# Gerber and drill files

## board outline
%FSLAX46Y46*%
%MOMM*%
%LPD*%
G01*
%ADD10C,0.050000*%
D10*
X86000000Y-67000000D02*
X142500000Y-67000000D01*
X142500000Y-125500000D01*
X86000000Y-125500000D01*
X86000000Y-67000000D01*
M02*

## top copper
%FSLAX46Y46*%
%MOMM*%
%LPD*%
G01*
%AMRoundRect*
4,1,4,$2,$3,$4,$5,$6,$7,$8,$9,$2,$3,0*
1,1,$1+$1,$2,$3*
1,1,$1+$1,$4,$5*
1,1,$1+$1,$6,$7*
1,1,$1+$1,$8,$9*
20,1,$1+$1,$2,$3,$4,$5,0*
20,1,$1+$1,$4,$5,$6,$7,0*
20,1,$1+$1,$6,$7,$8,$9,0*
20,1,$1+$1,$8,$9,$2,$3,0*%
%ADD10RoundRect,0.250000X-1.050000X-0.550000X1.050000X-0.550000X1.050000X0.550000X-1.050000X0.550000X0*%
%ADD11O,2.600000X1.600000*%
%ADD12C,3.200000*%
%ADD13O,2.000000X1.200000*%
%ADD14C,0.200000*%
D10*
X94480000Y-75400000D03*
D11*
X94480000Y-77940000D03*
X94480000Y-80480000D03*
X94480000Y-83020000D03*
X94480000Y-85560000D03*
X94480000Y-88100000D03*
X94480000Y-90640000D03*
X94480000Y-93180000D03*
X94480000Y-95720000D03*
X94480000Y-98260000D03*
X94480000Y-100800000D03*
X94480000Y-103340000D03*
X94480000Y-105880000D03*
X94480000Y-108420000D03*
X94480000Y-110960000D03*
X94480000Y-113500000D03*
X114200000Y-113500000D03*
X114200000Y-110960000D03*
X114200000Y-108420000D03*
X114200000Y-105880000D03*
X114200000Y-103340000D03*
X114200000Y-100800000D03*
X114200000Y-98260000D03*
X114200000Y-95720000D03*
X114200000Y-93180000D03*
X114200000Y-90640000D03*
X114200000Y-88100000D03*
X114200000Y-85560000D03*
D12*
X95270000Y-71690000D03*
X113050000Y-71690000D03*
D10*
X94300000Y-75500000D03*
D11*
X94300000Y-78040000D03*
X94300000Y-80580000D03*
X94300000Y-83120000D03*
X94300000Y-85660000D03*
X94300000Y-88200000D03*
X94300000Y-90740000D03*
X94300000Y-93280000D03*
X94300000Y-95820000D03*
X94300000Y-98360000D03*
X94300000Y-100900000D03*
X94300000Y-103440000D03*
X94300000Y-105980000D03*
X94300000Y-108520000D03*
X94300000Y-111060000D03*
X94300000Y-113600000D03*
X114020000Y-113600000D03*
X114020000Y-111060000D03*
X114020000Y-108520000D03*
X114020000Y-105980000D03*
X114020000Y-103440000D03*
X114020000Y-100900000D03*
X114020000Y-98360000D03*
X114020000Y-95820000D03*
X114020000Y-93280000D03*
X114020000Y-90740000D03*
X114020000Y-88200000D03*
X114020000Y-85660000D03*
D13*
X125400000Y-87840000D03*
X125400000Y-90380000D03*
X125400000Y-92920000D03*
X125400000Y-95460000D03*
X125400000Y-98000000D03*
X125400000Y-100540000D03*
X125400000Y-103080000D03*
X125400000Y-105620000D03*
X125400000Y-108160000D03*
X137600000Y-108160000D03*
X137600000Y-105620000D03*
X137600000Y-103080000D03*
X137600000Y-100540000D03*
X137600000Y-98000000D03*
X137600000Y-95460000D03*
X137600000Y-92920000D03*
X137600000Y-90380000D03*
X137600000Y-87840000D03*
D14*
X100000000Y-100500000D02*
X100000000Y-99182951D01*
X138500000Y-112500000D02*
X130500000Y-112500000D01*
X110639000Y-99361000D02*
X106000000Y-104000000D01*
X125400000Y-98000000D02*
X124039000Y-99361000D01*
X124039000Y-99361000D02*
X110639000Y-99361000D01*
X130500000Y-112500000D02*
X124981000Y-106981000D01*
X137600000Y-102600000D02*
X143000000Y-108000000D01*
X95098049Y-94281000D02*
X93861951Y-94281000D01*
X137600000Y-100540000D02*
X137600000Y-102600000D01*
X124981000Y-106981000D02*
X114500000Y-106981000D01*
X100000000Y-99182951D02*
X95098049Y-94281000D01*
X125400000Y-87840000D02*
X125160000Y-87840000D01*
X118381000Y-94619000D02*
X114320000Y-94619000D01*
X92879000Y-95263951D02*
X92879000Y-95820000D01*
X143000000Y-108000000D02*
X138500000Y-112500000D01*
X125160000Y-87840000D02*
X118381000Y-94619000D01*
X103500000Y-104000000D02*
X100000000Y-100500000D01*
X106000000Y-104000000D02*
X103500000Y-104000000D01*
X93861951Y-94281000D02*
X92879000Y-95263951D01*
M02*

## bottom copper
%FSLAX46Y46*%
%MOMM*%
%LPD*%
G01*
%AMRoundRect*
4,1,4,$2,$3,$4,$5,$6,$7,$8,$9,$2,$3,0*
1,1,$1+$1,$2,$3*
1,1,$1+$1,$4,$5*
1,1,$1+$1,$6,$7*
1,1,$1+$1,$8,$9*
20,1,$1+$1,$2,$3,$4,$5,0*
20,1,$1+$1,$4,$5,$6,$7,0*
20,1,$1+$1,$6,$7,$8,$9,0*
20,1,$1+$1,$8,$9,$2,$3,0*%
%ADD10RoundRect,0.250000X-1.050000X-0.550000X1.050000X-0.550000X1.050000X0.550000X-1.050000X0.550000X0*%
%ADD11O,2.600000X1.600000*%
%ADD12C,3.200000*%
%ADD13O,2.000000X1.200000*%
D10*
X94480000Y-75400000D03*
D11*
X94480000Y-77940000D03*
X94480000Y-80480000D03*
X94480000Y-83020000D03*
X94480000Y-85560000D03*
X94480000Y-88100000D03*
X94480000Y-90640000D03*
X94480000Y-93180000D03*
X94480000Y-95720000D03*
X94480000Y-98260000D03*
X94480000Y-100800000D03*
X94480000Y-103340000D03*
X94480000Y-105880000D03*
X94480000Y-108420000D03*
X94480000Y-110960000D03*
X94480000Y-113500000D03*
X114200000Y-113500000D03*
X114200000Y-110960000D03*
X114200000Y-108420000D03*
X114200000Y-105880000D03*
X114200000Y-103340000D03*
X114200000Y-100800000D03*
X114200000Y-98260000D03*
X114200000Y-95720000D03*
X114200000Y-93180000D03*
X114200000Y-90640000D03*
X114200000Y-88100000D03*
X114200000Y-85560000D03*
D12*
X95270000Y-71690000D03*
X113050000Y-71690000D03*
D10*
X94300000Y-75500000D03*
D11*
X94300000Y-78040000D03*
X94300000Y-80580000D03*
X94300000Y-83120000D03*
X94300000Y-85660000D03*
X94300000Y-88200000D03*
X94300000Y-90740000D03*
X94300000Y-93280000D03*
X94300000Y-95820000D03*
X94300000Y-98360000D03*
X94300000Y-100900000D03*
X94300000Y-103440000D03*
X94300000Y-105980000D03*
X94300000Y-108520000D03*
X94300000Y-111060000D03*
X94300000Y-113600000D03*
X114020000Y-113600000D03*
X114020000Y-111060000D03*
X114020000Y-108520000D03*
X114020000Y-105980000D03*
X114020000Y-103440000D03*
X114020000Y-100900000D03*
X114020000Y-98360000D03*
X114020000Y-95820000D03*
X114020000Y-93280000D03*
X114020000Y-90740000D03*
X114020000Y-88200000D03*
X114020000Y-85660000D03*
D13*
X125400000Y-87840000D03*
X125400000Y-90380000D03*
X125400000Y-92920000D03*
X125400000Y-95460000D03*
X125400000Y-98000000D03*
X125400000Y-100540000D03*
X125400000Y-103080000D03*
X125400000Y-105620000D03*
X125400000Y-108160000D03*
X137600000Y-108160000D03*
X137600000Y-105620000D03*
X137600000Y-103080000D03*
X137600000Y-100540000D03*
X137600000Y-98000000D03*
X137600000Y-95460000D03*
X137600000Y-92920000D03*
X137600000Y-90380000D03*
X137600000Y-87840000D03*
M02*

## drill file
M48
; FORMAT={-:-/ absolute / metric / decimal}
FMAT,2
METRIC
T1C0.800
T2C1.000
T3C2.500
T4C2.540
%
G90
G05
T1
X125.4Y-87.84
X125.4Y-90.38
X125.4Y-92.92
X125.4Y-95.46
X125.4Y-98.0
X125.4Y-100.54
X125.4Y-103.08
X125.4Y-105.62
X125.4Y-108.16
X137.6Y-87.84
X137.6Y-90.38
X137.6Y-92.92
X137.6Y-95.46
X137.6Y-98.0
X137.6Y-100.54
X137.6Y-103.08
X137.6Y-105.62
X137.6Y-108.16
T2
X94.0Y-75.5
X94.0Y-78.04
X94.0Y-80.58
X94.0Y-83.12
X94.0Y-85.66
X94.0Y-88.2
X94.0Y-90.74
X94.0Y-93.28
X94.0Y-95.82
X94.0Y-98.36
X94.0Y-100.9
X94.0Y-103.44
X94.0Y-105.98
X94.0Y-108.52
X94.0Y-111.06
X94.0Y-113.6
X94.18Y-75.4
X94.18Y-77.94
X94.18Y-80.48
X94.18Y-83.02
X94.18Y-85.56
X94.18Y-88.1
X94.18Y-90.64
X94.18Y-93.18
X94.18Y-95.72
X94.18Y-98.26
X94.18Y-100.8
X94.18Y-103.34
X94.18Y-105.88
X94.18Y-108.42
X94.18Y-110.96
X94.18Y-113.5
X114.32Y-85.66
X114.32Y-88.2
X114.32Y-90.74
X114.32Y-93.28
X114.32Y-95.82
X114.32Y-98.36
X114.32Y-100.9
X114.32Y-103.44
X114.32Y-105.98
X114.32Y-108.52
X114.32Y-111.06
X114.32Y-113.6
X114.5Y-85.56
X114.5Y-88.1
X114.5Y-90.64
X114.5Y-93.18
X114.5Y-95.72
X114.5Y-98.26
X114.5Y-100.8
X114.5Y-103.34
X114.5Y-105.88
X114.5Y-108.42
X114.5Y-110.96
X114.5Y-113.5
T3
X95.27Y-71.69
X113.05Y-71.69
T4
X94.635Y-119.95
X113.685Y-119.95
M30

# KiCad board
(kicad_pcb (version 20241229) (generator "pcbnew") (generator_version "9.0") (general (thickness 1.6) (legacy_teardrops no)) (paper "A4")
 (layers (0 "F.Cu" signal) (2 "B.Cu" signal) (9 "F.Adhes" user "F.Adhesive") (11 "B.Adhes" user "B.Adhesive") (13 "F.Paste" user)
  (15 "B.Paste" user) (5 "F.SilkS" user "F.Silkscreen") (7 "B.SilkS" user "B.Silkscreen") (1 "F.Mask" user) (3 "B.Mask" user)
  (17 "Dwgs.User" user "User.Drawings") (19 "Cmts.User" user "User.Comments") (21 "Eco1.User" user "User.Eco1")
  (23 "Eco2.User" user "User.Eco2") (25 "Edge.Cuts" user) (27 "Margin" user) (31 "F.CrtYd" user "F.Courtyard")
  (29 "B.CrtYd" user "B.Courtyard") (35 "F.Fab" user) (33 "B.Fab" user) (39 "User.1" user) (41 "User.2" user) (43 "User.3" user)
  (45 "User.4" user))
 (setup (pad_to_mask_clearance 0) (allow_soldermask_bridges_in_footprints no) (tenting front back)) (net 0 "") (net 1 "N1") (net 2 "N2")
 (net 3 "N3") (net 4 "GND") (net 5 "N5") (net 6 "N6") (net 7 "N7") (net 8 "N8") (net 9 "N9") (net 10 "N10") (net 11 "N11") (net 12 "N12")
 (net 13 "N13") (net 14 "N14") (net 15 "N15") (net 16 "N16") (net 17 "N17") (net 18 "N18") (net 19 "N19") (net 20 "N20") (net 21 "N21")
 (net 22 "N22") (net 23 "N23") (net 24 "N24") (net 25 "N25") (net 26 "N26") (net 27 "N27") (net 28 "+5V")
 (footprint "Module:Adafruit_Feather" (layer "F.Cu") (at 94.18 75.4)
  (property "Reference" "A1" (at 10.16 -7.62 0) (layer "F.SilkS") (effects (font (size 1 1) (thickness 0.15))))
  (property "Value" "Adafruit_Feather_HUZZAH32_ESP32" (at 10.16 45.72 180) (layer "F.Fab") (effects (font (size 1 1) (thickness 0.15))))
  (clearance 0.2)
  (pad "1" thru_hole roundrect (at 0 0) (size 2.6 1.6) (drill 1 (offset 0.3 0)) (layers "*.Cu" "*.Mask") (remove_unused_layers no)
   (roundrect_rratio 0.15625) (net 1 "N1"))
  (pad "2" thru_hole oval (at 0 2.54) (size 2.6 1.6) (drill 1 (offset 0.3 0)) (layers "*.Cu" "*.Mask") (remove_unused_layers no)
   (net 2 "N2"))
  (pad "3" thru_hole oval (at 0 5.08) (size 2.6 1.6) (drill 1 (offset 0.3 0)) (layers "*.Cu" "*.Mask") (remove_unused_layers no)
   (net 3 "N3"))
  (pad "4" thru_hole oval (at 0 7.62) (size 2.6 1.6) (drill 1 (offset 0.3 0)) (layers "*.Cu" "*.Mask") (remove_unused_layers no)
   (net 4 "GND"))
  (pad "5" thru_hole oval (at 0 10.16) (size 2.6 1.6) (drill 1 (offset 0.3 0)) (layers "*.Cu" "*.Mask") (remove_unused_layers no)
   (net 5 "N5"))
  (pad "6" thru_hole oval (at 0 12.7) (size 2.6 1.6) (drill 1 (offset 0.3 0)) (layers "*.Cu" "*.Mask") (remove_unused_layers no)
   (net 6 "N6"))
  (pad "7" thru_hole oval (at 0 15.24) (size 2.6 1.6) (drill 1 (offset 0.3 0)) (layers "*.Cu" "*.Mask") (remove_unused_layers no)
   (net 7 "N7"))
  (pad "8" thru_hole oval (at 0 17.78) (size 2.6 1.6) (drill 1 (offset 0.3 0)) (layers "*.Cu" "*.Mask") (remove_unused_layers no)
   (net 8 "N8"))
  (pad "9" thru_hole oval (at 0 20.32) (size 2.6 1.6) (drill 1 (offset 0.3 0)) (layers "*.Cu" "*.Mask") (remove_unused_layers no)
   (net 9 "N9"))
  (pad "10" thru_hole oval (at 0 22.86) (size 2.6 1.6) (drill 1 (offset 0.3 0)) (layers "*.Cu" "*.Mask") (remove_unused_layers no)
   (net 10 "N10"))
  (pad "11" thru_hole oval (at 0 25.4) (size 2.6 1.6) (drill 1 (offset 0.3 0)) (layers "*.Cu" "*.Mask") (remove_unused_layers no)
   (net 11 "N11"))
  (pad "12" thru_hole oval (at 0 27.94) (size 2.6 1.6) (drill 1 (offset 0.3 0)) (layers "*.Cu" "*.Mask") (remove_unused_layers no)
   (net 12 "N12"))
  (pad "13" thru_hole oval (at 0 30.48) (size 2.6 1.6) (drill 1 (offset 0.3 0)) (layers "*.Cu" "*.Mask") (remove_unused_layers no)
   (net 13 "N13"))
  (pad "14" thru_hole oval (at 0 33.02) (size 2.6 1.6) (drill 1 (offset 0.3 0)) (layers "*.Cu" "*.Mask") (remove_unused_layers no)
   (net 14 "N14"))
  (pad "15" thru_hole oval (at 0 35.56) (size 2.6 1.6) (drill 1 (offset 0.3 0)) (layers "*.Cu" "*.Mask") (remove_unused_layers no)
   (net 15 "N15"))
  (pad "16" thru_hole oval (at 0 38.1) (size 2.6 1.6) (drill 1 (offset 0.3 0)) (layers "*.Cu" "*.Mask") (remove_unused_layers no)
   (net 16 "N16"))
  (pad "17" thru_hole oval (at 20.32 38.1 180) (size 2.6 1.6) (drill 1 (offset 0.3 0)) (layers "*.Cu" "*.Mask") (remove_unused_layers no)
   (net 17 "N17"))
  (pad "18" thru_hole oval (at 20.32 35.56 180) (size 2.6 1.6) (drill 1 (offset 0.3 0)) (layers "*.Cu" "*.Mask") (remove_unused_layers no)
   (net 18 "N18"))
  (pad "19" thru_hole oval (at 20.32 33.02 180) (size 2.6 1.6) (drill 1 (offset 0.3 0)) (layers "*.Cu" "*.Mask") (remove_unused_layers no)
   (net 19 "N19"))
  (pad "20" thru_hole oval (at 20.32 30.48 180) (size 2.6 1.6) (drill 1 (offset 0.3 0)) (layers "*.Cu" "*.Mask") (remove_unused_layers no)
   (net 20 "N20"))
  (pad "21" thru_hole oval (at 20.32 27.94 180) (size 2.6 1.6) (drill 1 (offset 0.3 0)) (layers "*.Cu" "*.Mask") (remove_unused_layers no)
   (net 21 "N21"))
  (pad "22" thru_hole oval (at 20.32 25.4 180) (size 2.6 1.6) (drill 1 (offset 0.3 0)) (layers "*.Cu" "*.Mask") (remove_unused_layers no)
   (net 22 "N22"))
  (pad "23" thru_hole oval (at 20.32 22.86 180) (size 2.6 1.6) (drill 1 (offset 0.3 0)) (layers "*.Cu" "*.Mask") (remove_unused_layers no)
   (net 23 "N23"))
  (pad "24" thru_hole oval (at 20.32 20.32 180) (size 2.6 1.6) (drill 1 (offset 0.3 0)) (layers "*.Cu" "*.Mask") (remove_unused_layers no)
   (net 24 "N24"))
  (pad "25" thru_hole oval (at 20.32 17.78 180) (size 2.6 1.6) (drill 1 (offset 0.3 0)) (layers "*.Cu" "*.Mask") (remove_unused_layers no)
   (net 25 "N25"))
  (pad "26" thru_hole oval (at 20.32 15.24 180) (size 2.6 1.6) (drill 1 (offset 0.3 0)) (layers "*.Cu" "*.Mask") (remove_unused_layers no)
   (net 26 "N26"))
  (pad "27" thru_hole oval (at 20.32 12.7 180) (size 2.6 1.6) (drill 1 (offset 0.3 0)) (layers "*.Cu" "*.Mask") (remove_unused_layers no)
   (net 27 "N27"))
  (pad "28" thru_hole oval (at 20.32 10.16 180) (size 2.6 1.6) (drill 1 (offset 0.3 0)) (layers "*.Cu" "*.Mask") (remove_unused_layers no)
   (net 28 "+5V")))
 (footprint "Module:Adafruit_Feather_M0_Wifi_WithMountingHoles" (layer "F.Cu") (at 94 75.5)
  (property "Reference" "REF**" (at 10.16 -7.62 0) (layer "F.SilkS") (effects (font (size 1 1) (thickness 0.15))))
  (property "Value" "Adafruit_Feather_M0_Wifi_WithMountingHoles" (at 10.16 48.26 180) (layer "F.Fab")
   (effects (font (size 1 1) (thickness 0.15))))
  (pad "" np_thru_hole circle (at 0.635 44.45 270) (size 2.54 2.54) (drill 2.54) (layers "*.Cu" "*.Mask"))
  (pad "" np_thru_hole circle (at 1.27 -3.81 270) (size 3.2 3.2) (drill 2.5) (layers "*.Cu" "*.Mask"))
  (pad "" np_thru_hole circle (at 19.05 -3.81 270) (size 3.2 3.2) (drill 2.5) (layers "*.Cu" "*.Mask"))
  (pad "" np_thru_hole circle (at 19.685 44.45 270) (size 2.54 2.54) (drill 2.54) (layers "*.Cu" "*.Mask"))
  (pad "1" thru_hole roundrect (at 0 0) (size 2.6 1.6) (drill 1 (offset 0.3 0)) (layers "*.Cu" "*.Mask") (remove_unused_layers no)
   (roundrect_rratio 0.15625))
  (pad "2" thru_hole oval (at 0 2.54) (size 2.6 1.6) (drill 1 (offset 0.3 0)) (layers "*.Cu" "*.Mask") (remove_unused_layers no))
  (pad "3" thru_hole oval (at 0 5.08) (size 2.6 1.6) (drill 1 (offset 0.3 0)) (layers "*.Cu" "*.Mask") (remove_unused_layers no))
  (pad "4" thru_hole oval (at 0 7.62) (size 2.6 1.6) (drill 1 (offset 0.3 0)) (layers "*.Cu" "*.Mask") (remove_unused_layers no))
  (pad "5" thru_hole oval (at 0 10.16) (size 2.6 1.6) (drill 1 (offset 0.3 0)) (layers "*.Cu" "*.Mask") (remove_unused_layers no))
  (pad "6" thru_hole oval (at 0 12.7) (size 2.6 1.6) (drill 1 (offset 0.3 0)) (layers "*.Cu" "*.Mask") (remove_unused_layers no))
  (pad "7" thru_hole oval (at 0 15.24) (size 2.6 1.6) (drill 1 (offset 0.3 0)) (layers "*.Cu" "*.Mask") (remove_unused_layers no))
  (pad "8" thru_hole oval (at 0 17.78) (size 2.6 1.6) (drill 1 (offset 0.3 0)) (layers "*.Cu" "*.Mask") (remove_unused_layers no))
  (pad "9" thru_hole oval (at 0 20.32) (size 2.6 1.6) (drill 1 (offset 0.3 0)) (layers "*.Cu" "*.Mask") (remove_unused_layers no))
  (pad "10" thru_hole oval (at 0 22.86) (size 2.6 1.6) (drill 1 (offset 0.3 0)) (layers "*.Cu" "*.Mask") (remove_unused_layers no))
  (pad "11" thru_hole oval (at 0 25.4) (size 2.6 1.6) (drill 1 (offset 0.3 0)) (layers "*.Cu" "*.Mask") (remove_unused_layers no))
  (pad "12" thru_hole oval (at 0 27.94) (size 2.6 1.6) (drill 1 (offset 0.3 0)) (layers "*.Cu" "*.Mask") (remove_unused_layers no))
  (pad "13" thru_hole oval (at 0 30.48) (size 2.6 1.6) (drill 1 (offset 0.3 0)) (layers "*.Cu" "*.Mask") (remove_unused_layers no))
  (pad "14" thru_hole oval (at 0 33.02) (size 2.6 1.6) (drill 1 (offset 0.3 0)) (layers "*.Cu" "*.Mask") (remove_unused_layers no))
  (pad "15" thru_hole oval (at 0 35.56) (size 2.6 1.6) (drill 1 (offset 0.3 0)) (layers "*.Cu" "*.Mask") (remove_unused_layers no))
  (pad "16" thru_hole oval (at 0 38.1) (size 2.6 1.6) (drill 1 (offset 0.3 0)) (layers "*.Cu" "*.Mask") (remove_unused_layers no))
  (pad "17" thru_hole oval (at 20.32 38.1 180) (size 2.6 1.6) (drill 1 (offset 0.3 0)) (layers "*.Cu" "*.Mask") (remove_unused_layers no))
  (pad "18" thru_hole oval (at 20.32 35.56 180) (size 2.6 1.6) (drill 1 (offset 0.3 0)) (layers "*.Cu" "*.Mask") (remove_unused_layers no))
  (pad "19" thru_hole oval (at 20.32 33.02 180) (size 2.6 1.6) (drill 1 (offset 0.3 0)) (layers "*.Cu" "*.Mask") (remove_unused_layers no))
  (pad "20" thru_hole oval (at 20.32 30.48 180) (size 2.6 1.6) (drill 1 (offset 0.3 0)) (layers "*.Cu" "*.Mask") (remove_unused_layers no))
  (pad "21" thru_hole oval (at 20.32 27.94 180) (size 2.6 1.6) (drill 1 (offset 0.3 0)) (layers "*.Cu" "*.Mask") (remove_unused_layers no))
  (pad "22" thru_hole oval (at 20.32 25.4 180) (size 2.6 1.6) (drill 1 (offset 0.3 0)) (layers "*.Cu" "*.Mask") (remove_unused_layers no))
  (pad "23" thru_hole oval (at 20.32 22.86 180) (size 2.6 1.6) (drill 1 (offset 0.3 0)) (layers "*.Cu" "*.Mask") (remove_unused_layers no))
  (pad "24" thru_hole oval (at 20.32 20.32 180) (size 2.6 1.6) (drill 1 (offset 0.3 0)) (layers "*.Cu" "*.Mask") (remove_unused_layers no))
  (pad "25" thru_hole oval (at 20.32 17.78 180) (size 2.6 1.6) (drill 1 (offset 0.3 0)) (layers "*.Cu" "*.Mask") (remove_unused_layers no))
  (pad "26" thru_hole oval (at 20.32 15.24 180) (size 2.6 1.6) (drill 1 (offset 0.3 0)) (layers "*.Cu" "*.Mask") (remove_unused_layers no))
  (pad "27" thru_hole oval (at 20.32 12.7 180) (size 2.6 1.6) (drill 1 (offset 0.3 0)) (layers "*.Cu" "*.Mask") (remove_unused_layers no))
  (pad "28" thru_hole oval (at 20.32 10.16 180) (size 2.6 1.6) (drill 1 (offset 0.3 0)) (layers "*.Cu" "*.Mask") (remove_unused_layers no)))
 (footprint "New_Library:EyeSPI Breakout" (layer "F.Cu") (at 131.5 98 -90)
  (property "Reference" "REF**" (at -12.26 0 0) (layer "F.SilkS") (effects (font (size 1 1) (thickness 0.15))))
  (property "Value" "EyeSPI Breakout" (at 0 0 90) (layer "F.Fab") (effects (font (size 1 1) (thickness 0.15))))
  (pad "1" thru_hole oval (at -10.16 6.1 270) (size 1.2 2) (drill 0.8) (layers "*.Cu" "*.Mask") (remove_unused_layers no)
   (thermal_bridge_angle 45))
  (pad "2" thru_hole oval (at -7.62 6.1 270) (size 1.2 2) (drill 0.8) (layers "*.Cu" "*.Mask") (remove_unused_layers no)
   (thermal_bridge_angle 45))
  (pad "3" thru_hole oval (at -5.08 6.1 270) (size 1.2 2) (drill 0.8) (layers "*.Cu" "*.Mask") (remove_unused_layers no)
   (thermal_bridge_angle 45))
  (pad "4" thru_hole oval (at -2.54 6.1 270) (size 1.2 2) (drill 0.8) (layers "*.Cu" "*.Mask") (remove_unused_layers no)
   (thermal_bridge_angle 45))
  (pad "5" thru_hole oval (at 0 6.1 270) (size 1.2 2) (drill 0.8) (layers "*.Cu" "*.Mask") (remove_unused_layers no)
   (thermal_bridge_angle 45))
  (pad "6" thru_hole oval (at 2.54 6.1 270) (size 1.2 2) (drill 0.8) (layers "*.Cu" "*.Mask") (remove_unused_layers no)
   (thermal_bridge_angle 45))
  (pad "7" thru_hole oval (at 5.08 6.1 270) (size 1.2 2) (drill 0.8) (layers "*.Cu" "*.Mask") (remove_unused_layers no)
   (thermal_bridge_angle 45))
  (pad "8" thru_hole oval (at 7.62 6.1 270) (size 1.2 2) (drill 0.8) (layers "*.Cu" "*.Mask") (remove_unused_layers no)
   (thermal_bridge_angle 45))
  (pad "9" thru_hole oval (at 10.16 6.1 270) (size 1.2 2) (drill 0.8) (layers "*.Cu" "*.Mask") (remove_unused_layers no)
   (thermal_bridge_angle 45))
  (pad "10" thru_hole oval (at 10.16 -6.1 270) (size 1.2 2) (drill 0.8) (layers "*.Cu" "*.Mask") (remove_unused_layers no)
   (thermal_bridge_angle 45))
  (pad "11" thru_hole oval (at 7.62 -6.1 270) (size 1.2 2) (drill 0.8) (layers "*.Cu" "*.Mask") (remove_unused_layers no)
   (thermal_bridge_angle 45))
  (pad "12" thru_hole oval (at 5.08 -6.1 270) (size 1.2 2) (drill 0.8) (layers "*.Cu" "*.Mask") (remove_unused_layers no)
   (thermal_bridge_angle 45))
  (pad "13" thru_hole oval (at 2.54 -6.1 270) (size 1.2 2) (drill 0.8) (layers "*.Cu" "*.Mask") (remove_unused_layers no)
   (thermal_bridge_angle 45))
  (pad "14" thru_hole oval (at 0 -6.1 270) (size 1.2 2) (drill 0.8) (layers "*.Cu" "*.Mask") (remove_unused_layers no)
   (thermal_bridge_angle 45))
  (pad "15" thru_hole oval (at -2.54 -6.1 270) (size 1.2 2) (drill 0.8) (layers "*.Cu" "*.Mask") (remove_unused_layers no)
   (thermal_bridge_angle 45))
  (pad "16" thru_hole oval (at -5.08 -6.1 270) (size 1.2 2) (drill 0.8) (layers "*.Cu" "*.Mask") (remove_unused_layers no)
   (thermal_bridge_angle 45))
  (pad "17" thru_hole oval (at -7.62 -6.1 270) (size 1.2 2) (drill 0.8) (layers "*.Cu" "*.Mask") (remove_unused_layers no)
   (thermal_bridge_angle 45))
  (pad "18" thru_hole oval (at -10.16 -6.1 270) (size 1.2 2) (drill 0.8) (layers "*.Cu" "*.Mask") (remove_unused_layers no)
   (thermal_bridge_angle 45)))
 (gr_rect (start 86 67) (end 142.5 125.5) (stroke (width 0.05) (type default)) (fill no) (layer "Edge.Cuts"))
 (segment (start 100 100.5) (end 100 99.182951) (width 0.2) (layer "F.Cu") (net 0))
 (segment (start 138.5 112.5) (end 130.5 112.5) (width 0.2) (layer "F.Cu") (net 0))
 (segment (start 110.639 99.361) (end 106 104) (width 0.2) (layer "F.Cu") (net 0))
 (segment (start 125.4 98) (end 124.039 99.361) (width 0.2) (layer "F.Cu") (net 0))
 (segment (start 124.039 99.361) (end 110.639 99.361) (width 0.2) (layer "F.Cu") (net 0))
 (segment (start 130.5 112.5) (end 124.981 106.981) (width 0.2) (layer "F.Cu") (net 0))
 (segment (start 137.6 102.6) (end 143 108) (width 0.2) (layer "F.Cu") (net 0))
 (segment (start 95.098049 94.281) (end 93.861951 94.281) (width 0.2) (layer "F.Cu") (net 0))
 (segment (start 137.6 100.54) (end 137.6 102.6) (width 0.2) (layer "F.Cu") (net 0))
 (segment (start 124.981 106.981) (end 114.5 106.981) (width 0.2) (layer "F.Cu") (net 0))
 (segment (start 100 99.182951) (end 95.098049 94.281) (width 0.2) (layer "F.Cu") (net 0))
 (segment (start 125.4 87.84) (end 125.16 87.84) (width 0.2) (layer "F.Cu") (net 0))
 (segment (start 118.381 94.619) (end 114.32 94.619) (width 0.2) (layer "F.Cu") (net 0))
 (segment (start 92.879 95.263951) (end 92.879 95.82) (width 0.2) (layer "F.Cu") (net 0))
 (segment (start 143 108) (end 138.5 112.5) (width 0.2) (layer "F.Cu") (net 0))
 (segment (start 125.16 87.84) (end 118.381 94.619) (width 0.2) (layer "F.Cu") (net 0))
 (segment (start 103.5 104) (end 100 100.5) (width 0.2) (layer "F.Cu") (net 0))
 (segment (start 106 104) (end 103.5 104) (width 0.2) (layer "F.Cu") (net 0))
 (segment (start 93.861951 94.281) (end 92.879 95.263951) (width 0.2) (layer "F.Cu") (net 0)))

